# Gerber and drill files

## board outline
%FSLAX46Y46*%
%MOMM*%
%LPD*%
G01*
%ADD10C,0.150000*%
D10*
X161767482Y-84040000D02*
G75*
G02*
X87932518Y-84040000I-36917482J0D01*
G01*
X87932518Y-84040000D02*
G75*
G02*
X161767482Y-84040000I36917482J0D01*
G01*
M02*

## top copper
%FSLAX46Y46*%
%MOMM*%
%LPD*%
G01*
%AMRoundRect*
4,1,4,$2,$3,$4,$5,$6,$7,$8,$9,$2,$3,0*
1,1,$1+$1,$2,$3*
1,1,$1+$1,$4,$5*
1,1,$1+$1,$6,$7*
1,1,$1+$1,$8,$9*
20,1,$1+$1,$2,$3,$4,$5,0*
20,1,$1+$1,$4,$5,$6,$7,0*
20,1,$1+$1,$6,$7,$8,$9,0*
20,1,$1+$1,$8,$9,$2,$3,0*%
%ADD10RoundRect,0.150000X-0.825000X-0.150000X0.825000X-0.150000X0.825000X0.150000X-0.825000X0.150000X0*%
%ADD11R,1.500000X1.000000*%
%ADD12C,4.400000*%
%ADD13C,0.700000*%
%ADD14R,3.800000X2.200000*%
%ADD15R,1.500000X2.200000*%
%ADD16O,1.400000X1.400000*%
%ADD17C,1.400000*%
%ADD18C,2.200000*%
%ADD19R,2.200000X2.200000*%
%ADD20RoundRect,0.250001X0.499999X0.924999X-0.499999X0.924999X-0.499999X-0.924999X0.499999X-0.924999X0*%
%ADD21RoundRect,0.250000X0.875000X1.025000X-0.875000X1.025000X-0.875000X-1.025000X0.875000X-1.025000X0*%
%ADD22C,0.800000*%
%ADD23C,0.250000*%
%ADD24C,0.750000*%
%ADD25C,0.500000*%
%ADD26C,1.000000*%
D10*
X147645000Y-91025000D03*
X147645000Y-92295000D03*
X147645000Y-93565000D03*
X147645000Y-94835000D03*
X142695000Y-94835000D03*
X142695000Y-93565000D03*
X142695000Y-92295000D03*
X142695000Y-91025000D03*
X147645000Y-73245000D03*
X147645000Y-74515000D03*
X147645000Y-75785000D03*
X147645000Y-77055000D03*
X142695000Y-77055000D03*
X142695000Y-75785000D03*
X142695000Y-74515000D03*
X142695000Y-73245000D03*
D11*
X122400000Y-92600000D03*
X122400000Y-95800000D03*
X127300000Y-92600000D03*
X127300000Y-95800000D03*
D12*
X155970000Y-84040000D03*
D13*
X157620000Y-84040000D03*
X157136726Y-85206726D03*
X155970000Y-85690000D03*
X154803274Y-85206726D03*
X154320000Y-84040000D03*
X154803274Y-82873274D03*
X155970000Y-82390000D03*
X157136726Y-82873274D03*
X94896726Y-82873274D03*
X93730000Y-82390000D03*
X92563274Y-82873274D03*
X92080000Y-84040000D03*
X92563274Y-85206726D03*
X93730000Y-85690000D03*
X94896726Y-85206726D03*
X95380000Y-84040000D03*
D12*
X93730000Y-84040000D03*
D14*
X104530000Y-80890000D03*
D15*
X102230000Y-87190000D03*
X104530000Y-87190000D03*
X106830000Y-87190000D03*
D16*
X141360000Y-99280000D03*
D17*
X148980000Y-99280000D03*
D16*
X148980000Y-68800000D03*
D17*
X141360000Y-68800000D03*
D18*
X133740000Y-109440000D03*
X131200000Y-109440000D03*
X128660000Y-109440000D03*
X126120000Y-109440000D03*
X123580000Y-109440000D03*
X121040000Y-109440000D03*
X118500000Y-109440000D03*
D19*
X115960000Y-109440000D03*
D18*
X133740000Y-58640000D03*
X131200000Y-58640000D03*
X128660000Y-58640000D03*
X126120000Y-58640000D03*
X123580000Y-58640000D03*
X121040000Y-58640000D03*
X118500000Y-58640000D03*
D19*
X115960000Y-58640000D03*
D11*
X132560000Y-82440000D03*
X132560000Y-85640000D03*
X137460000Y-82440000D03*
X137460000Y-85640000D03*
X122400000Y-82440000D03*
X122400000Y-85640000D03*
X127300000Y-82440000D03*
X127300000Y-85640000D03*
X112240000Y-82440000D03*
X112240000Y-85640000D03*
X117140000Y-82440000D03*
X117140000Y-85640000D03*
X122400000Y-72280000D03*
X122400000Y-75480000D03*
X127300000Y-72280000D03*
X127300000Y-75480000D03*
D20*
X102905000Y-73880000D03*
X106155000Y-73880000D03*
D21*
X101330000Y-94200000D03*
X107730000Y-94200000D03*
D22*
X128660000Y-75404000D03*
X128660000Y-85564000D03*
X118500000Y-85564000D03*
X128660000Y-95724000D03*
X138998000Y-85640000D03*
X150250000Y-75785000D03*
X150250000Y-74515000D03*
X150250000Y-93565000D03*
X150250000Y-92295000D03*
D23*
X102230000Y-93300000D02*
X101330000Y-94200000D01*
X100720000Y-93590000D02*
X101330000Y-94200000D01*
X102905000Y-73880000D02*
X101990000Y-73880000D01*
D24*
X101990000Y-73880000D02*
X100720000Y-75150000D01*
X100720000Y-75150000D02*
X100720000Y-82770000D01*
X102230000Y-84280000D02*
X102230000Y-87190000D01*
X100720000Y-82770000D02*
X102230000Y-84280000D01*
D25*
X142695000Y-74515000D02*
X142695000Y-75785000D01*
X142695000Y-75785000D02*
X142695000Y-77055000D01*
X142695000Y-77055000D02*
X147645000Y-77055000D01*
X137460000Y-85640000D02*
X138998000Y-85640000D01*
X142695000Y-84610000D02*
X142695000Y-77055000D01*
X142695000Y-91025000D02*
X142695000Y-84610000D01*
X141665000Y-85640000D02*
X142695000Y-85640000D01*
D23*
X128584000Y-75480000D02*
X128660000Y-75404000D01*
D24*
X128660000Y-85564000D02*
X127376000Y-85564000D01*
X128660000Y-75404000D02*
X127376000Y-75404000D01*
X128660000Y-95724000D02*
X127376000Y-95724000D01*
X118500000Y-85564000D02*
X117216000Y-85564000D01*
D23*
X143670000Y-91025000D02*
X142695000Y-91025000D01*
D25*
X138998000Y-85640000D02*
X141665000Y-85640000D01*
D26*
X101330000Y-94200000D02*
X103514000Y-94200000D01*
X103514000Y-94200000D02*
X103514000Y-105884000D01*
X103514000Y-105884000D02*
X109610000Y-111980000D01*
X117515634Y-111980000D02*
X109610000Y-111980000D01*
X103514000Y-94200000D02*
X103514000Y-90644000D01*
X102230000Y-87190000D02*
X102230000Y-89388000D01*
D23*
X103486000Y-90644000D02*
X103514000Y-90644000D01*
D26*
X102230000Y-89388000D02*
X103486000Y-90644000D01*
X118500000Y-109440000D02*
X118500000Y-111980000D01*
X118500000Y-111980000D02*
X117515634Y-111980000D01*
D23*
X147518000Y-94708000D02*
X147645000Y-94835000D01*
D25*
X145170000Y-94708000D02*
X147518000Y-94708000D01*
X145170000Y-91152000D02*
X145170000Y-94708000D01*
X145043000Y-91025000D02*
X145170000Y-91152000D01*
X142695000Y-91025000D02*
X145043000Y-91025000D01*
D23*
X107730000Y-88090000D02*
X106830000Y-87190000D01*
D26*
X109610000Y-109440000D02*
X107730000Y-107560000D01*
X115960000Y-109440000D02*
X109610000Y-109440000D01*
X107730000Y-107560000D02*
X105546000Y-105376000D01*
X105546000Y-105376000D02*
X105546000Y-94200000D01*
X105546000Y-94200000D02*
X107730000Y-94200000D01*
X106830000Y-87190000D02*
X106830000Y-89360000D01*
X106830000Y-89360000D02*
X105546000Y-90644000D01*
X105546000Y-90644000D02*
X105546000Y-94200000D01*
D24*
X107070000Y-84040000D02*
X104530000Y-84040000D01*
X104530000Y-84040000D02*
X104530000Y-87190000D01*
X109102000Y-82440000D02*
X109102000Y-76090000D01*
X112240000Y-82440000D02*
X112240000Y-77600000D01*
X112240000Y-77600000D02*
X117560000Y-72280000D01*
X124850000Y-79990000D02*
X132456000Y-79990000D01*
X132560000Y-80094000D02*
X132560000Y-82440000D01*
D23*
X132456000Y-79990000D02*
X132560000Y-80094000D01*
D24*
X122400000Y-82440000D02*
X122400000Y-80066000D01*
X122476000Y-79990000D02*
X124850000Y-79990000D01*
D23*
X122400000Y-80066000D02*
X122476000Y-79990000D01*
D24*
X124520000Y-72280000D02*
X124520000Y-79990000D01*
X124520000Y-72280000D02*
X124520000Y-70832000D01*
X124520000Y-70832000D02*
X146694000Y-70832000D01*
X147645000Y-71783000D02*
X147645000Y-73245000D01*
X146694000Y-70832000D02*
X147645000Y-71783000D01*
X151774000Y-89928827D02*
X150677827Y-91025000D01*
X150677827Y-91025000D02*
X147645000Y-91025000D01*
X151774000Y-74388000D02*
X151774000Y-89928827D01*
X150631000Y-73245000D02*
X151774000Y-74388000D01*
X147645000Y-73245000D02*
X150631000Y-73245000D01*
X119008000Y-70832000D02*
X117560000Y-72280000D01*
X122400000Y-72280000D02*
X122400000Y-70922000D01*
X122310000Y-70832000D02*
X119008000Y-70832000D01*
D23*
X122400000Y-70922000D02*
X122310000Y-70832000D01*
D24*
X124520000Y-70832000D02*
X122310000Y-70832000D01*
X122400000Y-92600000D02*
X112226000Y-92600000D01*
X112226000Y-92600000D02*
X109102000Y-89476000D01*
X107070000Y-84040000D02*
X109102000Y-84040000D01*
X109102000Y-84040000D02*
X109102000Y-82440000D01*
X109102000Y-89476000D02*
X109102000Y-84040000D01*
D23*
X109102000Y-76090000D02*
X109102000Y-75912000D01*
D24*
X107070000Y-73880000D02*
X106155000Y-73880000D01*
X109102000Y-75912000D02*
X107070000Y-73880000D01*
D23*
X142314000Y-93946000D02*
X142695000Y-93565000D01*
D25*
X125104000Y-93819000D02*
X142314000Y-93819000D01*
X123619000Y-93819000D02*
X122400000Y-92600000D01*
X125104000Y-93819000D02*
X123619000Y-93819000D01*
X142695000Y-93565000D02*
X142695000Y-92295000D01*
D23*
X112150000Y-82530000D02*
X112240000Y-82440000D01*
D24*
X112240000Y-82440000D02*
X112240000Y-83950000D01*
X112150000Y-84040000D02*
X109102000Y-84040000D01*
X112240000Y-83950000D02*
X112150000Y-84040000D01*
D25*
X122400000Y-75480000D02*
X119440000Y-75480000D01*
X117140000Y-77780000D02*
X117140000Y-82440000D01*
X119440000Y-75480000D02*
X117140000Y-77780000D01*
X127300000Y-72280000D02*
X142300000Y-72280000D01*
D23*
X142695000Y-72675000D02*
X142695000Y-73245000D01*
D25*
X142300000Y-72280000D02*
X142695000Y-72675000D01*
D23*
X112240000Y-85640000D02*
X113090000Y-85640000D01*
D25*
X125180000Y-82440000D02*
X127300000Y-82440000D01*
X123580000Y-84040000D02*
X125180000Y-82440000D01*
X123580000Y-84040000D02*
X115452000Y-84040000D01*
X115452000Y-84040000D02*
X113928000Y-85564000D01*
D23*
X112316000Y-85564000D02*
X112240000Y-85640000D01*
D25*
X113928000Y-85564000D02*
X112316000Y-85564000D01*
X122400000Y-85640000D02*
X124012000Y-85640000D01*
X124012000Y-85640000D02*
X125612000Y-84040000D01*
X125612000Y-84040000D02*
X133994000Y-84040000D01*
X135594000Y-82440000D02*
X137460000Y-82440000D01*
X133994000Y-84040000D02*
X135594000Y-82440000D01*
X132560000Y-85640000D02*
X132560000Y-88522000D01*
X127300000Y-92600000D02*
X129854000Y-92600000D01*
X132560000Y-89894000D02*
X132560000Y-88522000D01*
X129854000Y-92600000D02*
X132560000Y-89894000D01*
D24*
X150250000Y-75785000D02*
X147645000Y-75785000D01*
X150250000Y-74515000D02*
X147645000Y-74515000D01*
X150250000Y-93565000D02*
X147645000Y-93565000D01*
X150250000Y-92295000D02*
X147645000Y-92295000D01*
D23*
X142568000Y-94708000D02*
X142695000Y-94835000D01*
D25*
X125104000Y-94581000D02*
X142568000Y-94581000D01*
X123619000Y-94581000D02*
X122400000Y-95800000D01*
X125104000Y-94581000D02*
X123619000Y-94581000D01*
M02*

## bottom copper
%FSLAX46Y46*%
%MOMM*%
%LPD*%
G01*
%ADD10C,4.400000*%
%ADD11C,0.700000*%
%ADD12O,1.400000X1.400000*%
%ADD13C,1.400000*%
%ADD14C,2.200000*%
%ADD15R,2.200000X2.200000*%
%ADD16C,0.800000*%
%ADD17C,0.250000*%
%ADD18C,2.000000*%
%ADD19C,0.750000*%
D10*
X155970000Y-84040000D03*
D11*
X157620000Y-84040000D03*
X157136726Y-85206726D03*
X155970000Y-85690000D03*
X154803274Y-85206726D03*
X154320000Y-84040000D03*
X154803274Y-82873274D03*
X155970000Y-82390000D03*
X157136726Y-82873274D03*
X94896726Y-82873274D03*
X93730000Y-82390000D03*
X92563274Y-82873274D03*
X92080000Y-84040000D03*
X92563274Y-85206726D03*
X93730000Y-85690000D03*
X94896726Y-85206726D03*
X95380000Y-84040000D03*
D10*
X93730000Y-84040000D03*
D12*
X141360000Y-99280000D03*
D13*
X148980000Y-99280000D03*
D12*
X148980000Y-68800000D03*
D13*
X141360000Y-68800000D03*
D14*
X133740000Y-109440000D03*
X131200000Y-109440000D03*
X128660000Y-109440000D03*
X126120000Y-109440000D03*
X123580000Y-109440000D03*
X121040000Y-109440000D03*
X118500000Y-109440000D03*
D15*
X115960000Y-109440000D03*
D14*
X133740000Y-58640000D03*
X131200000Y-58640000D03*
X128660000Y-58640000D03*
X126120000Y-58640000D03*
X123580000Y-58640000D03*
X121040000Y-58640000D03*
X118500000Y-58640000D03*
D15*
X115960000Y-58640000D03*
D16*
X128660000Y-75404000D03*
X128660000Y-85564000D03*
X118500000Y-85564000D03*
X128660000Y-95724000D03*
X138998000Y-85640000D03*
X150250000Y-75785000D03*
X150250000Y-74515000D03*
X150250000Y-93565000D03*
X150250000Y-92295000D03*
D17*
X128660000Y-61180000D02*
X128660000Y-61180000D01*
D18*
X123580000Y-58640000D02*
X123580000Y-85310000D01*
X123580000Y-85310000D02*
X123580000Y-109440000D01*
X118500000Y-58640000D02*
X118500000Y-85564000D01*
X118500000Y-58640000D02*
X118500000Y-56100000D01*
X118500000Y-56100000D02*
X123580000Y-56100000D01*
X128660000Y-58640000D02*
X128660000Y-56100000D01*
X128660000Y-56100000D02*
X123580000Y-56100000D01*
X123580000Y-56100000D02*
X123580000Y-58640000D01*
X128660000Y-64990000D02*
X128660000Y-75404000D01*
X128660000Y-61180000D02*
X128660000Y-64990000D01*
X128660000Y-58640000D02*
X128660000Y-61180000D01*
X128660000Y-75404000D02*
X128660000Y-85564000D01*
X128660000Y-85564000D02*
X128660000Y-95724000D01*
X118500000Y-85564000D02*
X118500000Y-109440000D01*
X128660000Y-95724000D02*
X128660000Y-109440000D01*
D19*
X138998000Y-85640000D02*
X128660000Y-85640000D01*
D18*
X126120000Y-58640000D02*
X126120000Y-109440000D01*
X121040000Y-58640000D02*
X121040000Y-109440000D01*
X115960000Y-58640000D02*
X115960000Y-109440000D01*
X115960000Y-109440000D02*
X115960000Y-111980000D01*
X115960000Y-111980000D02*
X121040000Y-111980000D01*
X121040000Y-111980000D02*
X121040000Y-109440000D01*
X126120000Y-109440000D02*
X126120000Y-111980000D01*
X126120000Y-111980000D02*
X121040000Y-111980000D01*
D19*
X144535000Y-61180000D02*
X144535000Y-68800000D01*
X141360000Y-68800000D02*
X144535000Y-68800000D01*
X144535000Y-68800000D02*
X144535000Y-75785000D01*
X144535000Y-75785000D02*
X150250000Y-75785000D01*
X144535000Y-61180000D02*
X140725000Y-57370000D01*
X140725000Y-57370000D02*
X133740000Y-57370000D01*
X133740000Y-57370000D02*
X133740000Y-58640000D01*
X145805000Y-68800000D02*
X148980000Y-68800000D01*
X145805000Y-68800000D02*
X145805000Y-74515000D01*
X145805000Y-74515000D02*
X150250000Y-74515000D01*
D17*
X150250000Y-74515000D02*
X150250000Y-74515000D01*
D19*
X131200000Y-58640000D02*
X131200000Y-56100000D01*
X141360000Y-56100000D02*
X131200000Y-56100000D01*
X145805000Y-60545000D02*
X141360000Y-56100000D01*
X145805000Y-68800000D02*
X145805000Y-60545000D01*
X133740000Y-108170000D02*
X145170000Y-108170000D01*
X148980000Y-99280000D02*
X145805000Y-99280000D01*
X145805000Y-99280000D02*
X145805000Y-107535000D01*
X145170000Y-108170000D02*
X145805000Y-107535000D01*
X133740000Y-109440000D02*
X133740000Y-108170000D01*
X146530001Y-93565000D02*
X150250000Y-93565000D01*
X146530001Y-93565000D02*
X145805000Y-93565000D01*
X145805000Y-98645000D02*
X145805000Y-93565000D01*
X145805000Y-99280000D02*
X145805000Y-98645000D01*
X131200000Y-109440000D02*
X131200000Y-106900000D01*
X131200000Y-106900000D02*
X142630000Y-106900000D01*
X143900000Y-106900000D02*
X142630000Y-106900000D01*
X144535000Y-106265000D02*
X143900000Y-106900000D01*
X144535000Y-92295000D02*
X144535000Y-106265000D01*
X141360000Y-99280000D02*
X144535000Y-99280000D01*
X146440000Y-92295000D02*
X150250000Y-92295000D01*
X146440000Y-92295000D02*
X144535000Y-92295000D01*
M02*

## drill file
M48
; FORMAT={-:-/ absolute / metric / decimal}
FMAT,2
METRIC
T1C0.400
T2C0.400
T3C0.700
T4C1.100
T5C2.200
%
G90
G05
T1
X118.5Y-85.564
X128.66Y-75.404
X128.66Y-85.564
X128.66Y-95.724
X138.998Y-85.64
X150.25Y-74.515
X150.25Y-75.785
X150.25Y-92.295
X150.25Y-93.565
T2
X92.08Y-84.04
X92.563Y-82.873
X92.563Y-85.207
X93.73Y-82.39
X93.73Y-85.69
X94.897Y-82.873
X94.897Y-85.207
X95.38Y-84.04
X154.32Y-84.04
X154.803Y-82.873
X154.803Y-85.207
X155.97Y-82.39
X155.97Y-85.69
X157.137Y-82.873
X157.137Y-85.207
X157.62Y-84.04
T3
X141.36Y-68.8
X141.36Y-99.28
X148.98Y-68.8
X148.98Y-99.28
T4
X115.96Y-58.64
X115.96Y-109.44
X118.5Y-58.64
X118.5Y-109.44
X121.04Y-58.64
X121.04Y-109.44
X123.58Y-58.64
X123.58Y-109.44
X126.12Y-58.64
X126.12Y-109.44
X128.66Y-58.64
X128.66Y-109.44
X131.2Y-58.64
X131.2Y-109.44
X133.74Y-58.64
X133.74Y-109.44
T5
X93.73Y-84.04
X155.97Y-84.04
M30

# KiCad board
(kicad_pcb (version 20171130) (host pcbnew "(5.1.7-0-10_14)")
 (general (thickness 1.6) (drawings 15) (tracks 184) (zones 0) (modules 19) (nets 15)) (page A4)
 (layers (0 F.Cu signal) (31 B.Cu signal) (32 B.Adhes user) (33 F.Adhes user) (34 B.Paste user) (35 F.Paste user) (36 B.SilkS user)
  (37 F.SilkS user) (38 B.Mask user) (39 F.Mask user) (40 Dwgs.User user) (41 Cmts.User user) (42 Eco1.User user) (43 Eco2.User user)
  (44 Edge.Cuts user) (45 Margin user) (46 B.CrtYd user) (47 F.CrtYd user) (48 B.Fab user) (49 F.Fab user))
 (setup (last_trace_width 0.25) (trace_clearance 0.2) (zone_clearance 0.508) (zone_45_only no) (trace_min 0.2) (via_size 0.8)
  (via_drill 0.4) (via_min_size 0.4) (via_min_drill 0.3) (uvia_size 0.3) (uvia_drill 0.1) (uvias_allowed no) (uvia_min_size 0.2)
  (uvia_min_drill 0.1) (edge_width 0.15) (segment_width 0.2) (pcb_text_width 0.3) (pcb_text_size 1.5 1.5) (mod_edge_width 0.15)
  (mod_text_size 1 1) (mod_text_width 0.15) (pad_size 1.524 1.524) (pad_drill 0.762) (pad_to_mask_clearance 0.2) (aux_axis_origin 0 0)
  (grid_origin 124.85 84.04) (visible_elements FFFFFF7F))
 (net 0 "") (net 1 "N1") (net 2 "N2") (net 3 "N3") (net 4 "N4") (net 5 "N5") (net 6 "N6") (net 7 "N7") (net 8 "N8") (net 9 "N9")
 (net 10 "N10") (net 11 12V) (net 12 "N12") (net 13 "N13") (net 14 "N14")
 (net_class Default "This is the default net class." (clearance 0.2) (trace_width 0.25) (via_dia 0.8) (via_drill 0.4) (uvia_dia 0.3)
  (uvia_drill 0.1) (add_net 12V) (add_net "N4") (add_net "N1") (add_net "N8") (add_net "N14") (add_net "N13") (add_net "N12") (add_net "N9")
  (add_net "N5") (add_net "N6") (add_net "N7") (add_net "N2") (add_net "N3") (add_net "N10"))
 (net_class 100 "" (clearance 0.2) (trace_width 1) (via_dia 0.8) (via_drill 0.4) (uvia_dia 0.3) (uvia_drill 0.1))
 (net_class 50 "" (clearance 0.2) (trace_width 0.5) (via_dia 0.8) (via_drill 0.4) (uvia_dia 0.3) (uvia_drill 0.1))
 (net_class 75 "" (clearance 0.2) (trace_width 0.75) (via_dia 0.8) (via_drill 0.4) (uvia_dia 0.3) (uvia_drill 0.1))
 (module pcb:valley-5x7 (layer F.Cu) (at 116.468 102.836)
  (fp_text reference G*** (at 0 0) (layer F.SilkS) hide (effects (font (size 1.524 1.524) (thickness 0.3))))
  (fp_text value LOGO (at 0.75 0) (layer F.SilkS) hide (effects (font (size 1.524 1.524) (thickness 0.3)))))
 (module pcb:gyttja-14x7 (layer F.Cu) (at 127.39 102.836)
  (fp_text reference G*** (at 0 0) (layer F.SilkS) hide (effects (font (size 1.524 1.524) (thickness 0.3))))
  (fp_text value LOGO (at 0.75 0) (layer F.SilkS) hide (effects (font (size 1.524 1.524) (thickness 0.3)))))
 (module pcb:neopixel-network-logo (layer F.Cu) (at 125.104 64.736)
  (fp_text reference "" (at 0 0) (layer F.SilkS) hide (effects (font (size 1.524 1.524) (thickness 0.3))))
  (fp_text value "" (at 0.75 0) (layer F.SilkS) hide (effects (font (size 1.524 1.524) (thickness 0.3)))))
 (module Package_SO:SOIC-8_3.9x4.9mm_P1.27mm (layer F.Cu) (at 145.17 92.93)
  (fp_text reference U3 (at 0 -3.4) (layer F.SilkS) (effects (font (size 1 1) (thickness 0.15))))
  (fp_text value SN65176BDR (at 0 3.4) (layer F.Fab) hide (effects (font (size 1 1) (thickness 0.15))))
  (pad 8 smd roundrect (at 2.475 -1.905) (size 1.95 0.6) (layers F.Cu F.Paste F.Mask) (roundrect_rratio 0.25) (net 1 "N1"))
  (pad 7 smd roundrect (at 2.475 -0.635) (size 1.95 0.6) (layers F.Cu F.Paste F.Mask) (roundrect_rratio 0.25) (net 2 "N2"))
  (pad 6 smd roundrect (at 2.475 0.635) (size 1.95 0.6) (layers F.Cu F.Paste F.Mask) (roundrect_rratio 0.25) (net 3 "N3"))
  (pad 5 smd roundrect (at 2.475 1.905) (size 1.95 0.6) (layers F.Cu F.Paste F.Mask) (roundrect_rratio 0.25) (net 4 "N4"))
  (pad 4 smd roundrect (at -2.475 1.905) (size 1.95 0.6) (layers F.Cu F.Paste F.Mask) (roundrect_rratio 0.25) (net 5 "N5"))
  (pad 3 smd roundrect (at -2.475 0.635) (size 1.95 0.6) (layers F.Cu F.Paste F.Mask) (roundrect_rratio 0.25) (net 1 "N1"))
  (pad 2 smd roundrect (at -2.475 -0.635) (size 1.95 0.6) (layers F.Cu F.Paste F.Mask) (roundrect_rratio 0.25) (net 1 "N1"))
  (pad 1 smd roundrect (at -2.475 -1.905) (size 1.95 0.6) (layers F.Cu F.Paste F.Mask) (roundrect_rratio 0.25) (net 4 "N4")))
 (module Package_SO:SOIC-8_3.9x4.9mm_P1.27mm (layer F.Cu) (at 145.17 75.15)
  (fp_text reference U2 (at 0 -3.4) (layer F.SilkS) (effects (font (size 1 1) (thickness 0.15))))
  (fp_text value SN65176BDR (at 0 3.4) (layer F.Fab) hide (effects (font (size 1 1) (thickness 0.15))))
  (pad 8 smd roundrect (at 2.475 -1.905) (size 1.95 0.6) (layers F.Cu F.Paste F.Mask) (roundrect_rratio 0.25) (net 1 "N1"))
  (pad 7 smd roundrect (at 2.475 -0.635) (size 1.95 0.6) (layers F.Cu F.Paste F.Mask) (roundrect_rratio 0.25) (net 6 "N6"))
  (pad 6 smd roundrect (at 2.475 0.635) (size 1.95 0.6) (layers F.Cu F.Paste F.Mask) (roundrect_rratio 0.25) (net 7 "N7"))
  (pad 5 smd roundrect (at 2.475 1.905) (size 1.95 0.6) (layers F.Cu F.Paste F.Mask) (roundrect_rratio 0.25) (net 4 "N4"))
  (pad 4 smd roundrect (at -2.475 1.905) (size 1.95 0.6) (layers F.Cu F.Paste F.Mask) (roundrect_rratio 0.25) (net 4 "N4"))
  (pad 3 smd roundrect (at -2.475 0.635) (size 1.95 0.6) (layers F.Cu F.Paste F.Mask) (roundrect_rratio 0.25) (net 4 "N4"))
  (pad 2 smd roundrect (at -2.475 -0.635) (size 1.95 0.6) (layers F.Cu F.Paste F.Mask) (roundrect_rratio 0.25) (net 4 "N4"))
  (pad 1 smd roundrect (at -2.475 -1.905) (size 1.95 0.6) (layers F.Cu F.Paste F.Mask) (roundrect_rratio 0.25) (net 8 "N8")))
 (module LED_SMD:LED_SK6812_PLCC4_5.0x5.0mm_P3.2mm (layer F.Cu) (at 124.85 94.2)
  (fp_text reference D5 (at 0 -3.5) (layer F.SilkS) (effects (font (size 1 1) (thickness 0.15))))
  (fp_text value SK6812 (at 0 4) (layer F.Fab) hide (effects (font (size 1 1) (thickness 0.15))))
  (pad 3 smd rect (at -2.45 -1.6) (size 1.5 1) (layers F.Cu F.Paste F.Mask) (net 1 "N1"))
  (pad 4 smd rect (at -2.45 1.6) (size 1.5 1) (layers F.Cu F.Paste F.Mask) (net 5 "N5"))
  (pad 2 smd rect (at 2.45 -1.6) (size 1.5 1) (layers F.Cu F.Paste F.Mask) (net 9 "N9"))
  (pad 1 smd rect (at 2.45 1.6) (size 1.5 1) (layers F.Cu F.Paste F.Mask) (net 4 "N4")))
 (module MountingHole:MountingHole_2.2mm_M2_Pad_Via (layer F.Cu) (at 155.97 84.04)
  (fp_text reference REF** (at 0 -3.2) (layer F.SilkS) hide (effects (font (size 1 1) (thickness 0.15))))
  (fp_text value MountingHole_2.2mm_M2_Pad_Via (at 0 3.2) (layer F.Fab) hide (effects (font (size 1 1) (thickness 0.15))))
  (pad 1 thru_hole circle (at 0 0) (size 4.4 4.4) (drill 2.2) (layers *.Cu *.Mask))
  (pad 1 thru_hole circle (at 1.65 0) (size 0.7 0.7) (drill 0.4) (layers *.Cu *.Mask))
  (pad 1 thru_hole circle (at 1.166726 1.166726) (size 0.7 0.7) (drill 0.4) (layers *.Cu *.Mask))
  (pad 1 thru_hole circle (at 0 1.65) (size 0.7 0.7) (drill 0.4) (layers *.Cu *.Mask))
  (pad 1 thru_hole circle (at -1.166726 1.166726) (size 0.7 0.7) (drill 0.4) (layers *.Cu *.Mask))
  (pad 1 thru_hole circle (at -1.65 0) (size 0.7 0.7) (drill 0.4) (layers *.Cu *.Mask))
  (pad 1 thru_hole circle (at -1.166726 -1.166726) (size 0.7 0.7) (drill 0.4) (layers *.Cu *.Mask))
  (pad 1 thru_hole circle (at 0 -1.65) (size 0.7 0.7) (drill 0.4) (layers *.Cu *.Mask))
  (pad 1 thru_hole circle (at 1.166726 -1.166726) (size 0.7 0.7) (drill 0.4) (layers *.Cu *.Mask)))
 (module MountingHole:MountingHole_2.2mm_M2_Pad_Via (layer F.Cu) (at 93.73 84.04)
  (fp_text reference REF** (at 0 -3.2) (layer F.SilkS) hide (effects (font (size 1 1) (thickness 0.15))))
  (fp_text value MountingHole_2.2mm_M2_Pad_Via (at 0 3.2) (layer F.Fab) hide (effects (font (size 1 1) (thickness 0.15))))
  (pad 1 thru_hole circle (at 1.166726 -1.166726) (size 0.7 0.7) (drill 0.4) (layers *.Cu *.Mask))
  (pad 1 thru_hole circle (at 0 -1.65) (size 0.7 0.7) (drill 0.4) (layers *.Cu *.Mask))
  (pad 1 thru_hole circle (at -1.166726 -1.166726) (size 0.7 0.7) (drill 0.4) (layers *.Cu *.Mask))
  (pad 1 thru_hole circle (at -1.65 0) (size 0.7 0.7) (drill 0.4) (layers *.Cu *.Mask))
  (pad 1 thru_hole circle (at -1.166726 1.166726) (size 0.7 0.7) (drill 0.4) (layers *.Cu *.Mask))
  (pad 1 thru_hole circle (at 0 1.65) (size 0.7 0.7) (drill 0.4) (layers *.Cu *.Mask))
  (pad 1 thru_hole circle (at 1.166726 1.166726) (size 0.7 0.7) (drill 0.4) (layers *.Cu *.Mask))
  (pad 1 thru_hole circle (at 1.65 0) (size 0.7 0.7) (drill 0.4) (layers *.Cu *.Mask))
  (pad 1 thru_hole circle (at 0 0) (size 4.4 4.4) (drill 2.2) (layers *.Cu *.Mask)))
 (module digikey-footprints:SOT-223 (layer F.Cu) (at 104.53 84.04)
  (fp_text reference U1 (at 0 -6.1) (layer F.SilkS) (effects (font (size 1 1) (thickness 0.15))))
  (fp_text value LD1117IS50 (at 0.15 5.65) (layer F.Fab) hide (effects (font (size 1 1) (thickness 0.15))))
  (pad 4 smd rect (at 0 -3.15) (size 3.8 2.2) (layers F.Cu F.Paste F.Mask) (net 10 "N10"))
  (pad 1 smd rect (at -2.3 3.15) (size 1.5 2.2) (layers F.Cu F.Paste F.Mask) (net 4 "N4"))
  (pad 2 smd rect (at 0 3.15) (size 1.5 2.2) (layers F.Cu F.Paste F.Mask) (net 1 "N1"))
  (pad 3 smd rect (at 2.3 3.15) (size 1.5 2.2) (layers F.Cu F.Paste F.Mask) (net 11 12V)))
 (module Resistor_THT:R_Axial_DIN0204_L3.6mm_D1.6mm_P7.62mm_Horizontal (layer F.Cu) (at 148.98 99.28 180)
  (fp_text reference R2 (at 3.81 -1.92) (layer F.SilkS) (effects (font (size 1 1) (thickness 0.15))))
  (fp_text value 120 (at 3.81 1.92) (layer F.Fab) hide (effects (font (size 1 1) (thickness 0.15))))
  (pad 2 thru_hole oval (at 7.62 0 180) (size 1.4 1.4) (drill 0.7) (layers *.Cu *.Mask) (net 2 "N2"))
  (pad 1 thru_hole circle (at 0 0 180) (size 1.4 1.4) (drill 0.7) (layers *.Cu *.Mask) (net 3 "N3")))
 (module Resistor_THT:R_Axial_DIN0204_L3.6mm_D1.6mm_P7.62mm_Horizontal (layer F.Cu) (at 141.36 68.8)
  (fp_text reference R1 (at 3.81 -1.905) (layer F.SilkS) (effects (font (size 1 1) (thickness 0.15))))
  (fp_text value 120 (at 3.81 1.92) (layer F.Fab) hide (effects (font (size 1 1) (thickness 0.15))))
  (pad 2 thru_hole oval (at 7.62 0) (size 1.4 1.4) (drill 0.7) (layers *.Cu *.Mask) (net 6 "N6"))
  (pad 1 thru_hole circle (at 0 0) (size 1.4 1.4) (drill 0.7) (layers *.Cu *.Mask) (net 7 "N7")))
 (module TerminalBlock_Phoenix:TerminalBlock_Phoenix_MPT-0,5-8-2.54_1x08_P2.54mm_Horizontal (layer B.Cu) (at 115.96 109.44)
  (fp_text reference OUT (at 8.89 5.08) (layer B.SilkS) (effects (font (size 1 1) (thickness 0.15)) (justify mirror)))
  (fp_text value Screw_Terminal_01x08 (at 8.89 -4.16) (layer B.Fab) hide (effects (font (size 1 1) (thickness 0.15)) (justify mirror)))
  (pad 8 thru_hole circle (at 17.78 0) (size 2.2 2.2) (drill 1.1) (layers *.Cu *.Mask) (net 3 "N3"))
  (pad 7 thru_hole circle (at 15.24 0) (size 2.2 2.2) (drill 1.1) (layers *.Cu *.Mask) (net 2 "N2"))
  (pad 6 thru_hole circle (at 12.7 0) (size 2.2 2.2) (drill 1.1) (layers *.Cu *.Mask) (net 4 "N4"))
  (pad 5 thru_hole circle (at 10.16 0) (size 2.2 2.2) (drill 1.1) (layers *.Cu *.Mask) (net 11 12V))
  (pad 4 thru_hole circle (at 7.62 0) (size 2.2 2.2) (drill 1.1) (layers *.Cu *.Mask) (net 4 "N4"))
  (pad 3 thru_hole circle (at 5.08 0) (size 2.2 2.2) (drill 1.1) (layers *.Cu *.Mask) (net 11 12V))
  (pad 2 thru_hole circle (at 2.54 0) (size 2.2 2.2) (drill 1.1) (layers *.Cu *.Mask) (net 4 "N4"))
  (pad 1 thru_hole rect (at 0 0) (size 2.2 2.2) (drill 1.1) (layers *.Cu *.Mask) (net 11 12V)))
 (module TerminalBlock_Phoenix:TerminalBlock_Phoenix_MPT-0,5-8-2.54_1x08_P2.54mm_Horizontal (layer B.Cu) (at 115.96 58.64)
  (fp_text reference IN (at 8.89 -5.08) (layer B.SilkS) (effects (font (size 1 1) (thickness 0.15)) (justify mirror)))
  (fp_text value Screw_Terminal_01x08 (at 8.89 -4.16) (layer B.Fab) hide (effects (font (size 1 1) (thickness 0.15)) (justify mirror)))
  (pad 8 thru_hole circle (at 17.78 0) (size 2.2 2.2) (drill 1.1) (layers *.Cu *.Mask) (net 7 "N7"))
  (pad 7 thru_hole circle (at 15.24 0) (size 2.2 2.2) (drill 1.1) (layers *.Cu *.Mask) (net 6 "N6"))
  (pad 6 thru_hole circle (at 12.7 0) (size 2.2 2.2) (drill 1.1) (layers *.Cu *.Mask) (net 4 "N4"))
  (pad 5 thru_hole circle (at 10.16 0) (size 2.2 2.2) (drill 1.1) (layers *.Cu *.Mask) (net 11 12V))
  (pad 4 thru_hole circle (at 7.62 0) (size 2.2 2.2) (drill 1.1) (layers *.Cu *.Mask) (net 4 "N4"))
  (pad 3 thru_hole circle (at 5.08 0) (size 2.2 2.2) (drill 1.1) (layers *.Cu *.Mask) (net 11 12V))
  (pad 2 thru_hole circle (at 2.54 0) (size 2.2 2.2) (drill 1.1) (layers *.Cu *.Mask) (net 4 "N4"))
  (pad 1 thru_hole rect (at 0 0) (size 2.2 2.2) (drill 1.1) (layers *.Cu *.Mask) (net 11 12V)))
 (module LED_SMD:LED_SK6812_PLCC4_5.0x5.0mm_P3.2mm (layer F.Cu) (at 135.01 84.04)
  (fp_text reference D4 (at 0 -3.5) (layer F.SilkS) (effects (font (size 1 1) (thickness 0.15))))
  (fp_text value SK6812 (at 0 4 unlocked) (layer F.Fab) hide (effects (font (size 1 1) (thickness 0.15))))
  (pad 3 smd rect (at -2.45 -1.6) (size 1.5 1) (layers F.Cu F.Paste F.Mask) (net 1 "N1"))
  (pad 4 smd rect (at -2.45 1.6) (size 1.5 1) (layers F.Cu F.Paste F.Mask) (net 9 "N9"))
  (pad 2 smd rect (at 2.45 -1.6) (size 1.5 1) (layers F.Cu F.Paste F.Mask) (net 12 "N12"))
  (pad 1 smd rect (at 2.45 1.6) (size 1.5 1) (layers F.Cu F.Paste F.Mask) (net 4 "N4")))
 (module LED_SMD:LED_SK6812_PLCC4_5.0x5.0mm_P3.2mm (layer F.Cu) (at 124.85 84.04)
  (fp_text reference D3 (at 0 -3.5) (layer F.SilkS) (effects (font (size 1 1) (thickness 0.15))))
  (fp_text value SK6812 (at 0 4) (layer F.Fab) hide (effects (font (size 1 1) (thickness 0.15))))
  (pad 3 smd rect (at -2.45 -1.6) (size 1.5 1) (layers F.Cu F.Paste F.Mask) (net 1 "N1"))
  (pad 4 smd rect (at -2.45 1.6) (size 1.5 1) (layers F.Cu F.Paste F.Mask) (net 12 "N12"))
  (pad 2 smd rect (at 2.45 -1.6) (size 1.5 1) (layers F.Cu F.Paste F.Mask) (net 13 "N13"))
  (pad 1 smd rect (at 2.45 1.6) (size 1.5 1) (layers F.Cu F.Paste F.Mask) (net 4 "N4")))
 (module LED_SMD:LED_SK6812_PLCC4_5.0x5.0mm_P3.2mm (layer F.Cu) (at 114.69 84.04)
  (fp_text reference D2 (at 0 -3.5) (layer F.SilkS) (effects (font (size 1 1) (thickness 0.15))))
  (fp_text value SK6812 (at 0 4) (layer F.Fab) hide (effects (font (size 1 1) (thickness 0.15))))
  (pad 3 smd rect (at -2.45 -1.6) (size 1.5 1) (layers F.Cu F.Paste F.Mask) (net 1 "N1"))
  (pad 4 smd rect (at -2.45 1.6) (size 1.5 1) (layers F.Cu F.Paste F.Mask) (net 13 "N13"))
  (pad 2 smd rect (at 2.45 -1.6) (size 1.5 1) (layers F.Cu F.Paste F.Mask) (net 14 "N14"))
  (pad 1 smd rect (at 2.45 1.6) (size 1.5 1) (layers F.Cu F.Paste F.Mask) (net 4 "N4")))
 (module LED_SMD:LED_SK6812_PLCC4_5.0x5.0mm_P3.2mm (layer F.Cu) (at 124.85 73.88)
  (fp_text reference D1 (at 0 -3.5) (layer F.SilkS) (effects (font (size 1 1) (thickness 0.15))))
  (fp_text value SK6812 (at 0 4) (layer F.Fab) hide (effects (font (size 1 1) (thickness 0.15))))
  (pad 3 smd rect (at -2.45 -1.6) (size 1.5 1) (layers F.Cu F.Paste F.Mask) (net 1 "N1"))
  (pad 4 smd rect (at -2.45 1.6) (size 1.5 1) (layers F.Cu F.Paste F.Mask) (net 14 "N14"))
  (pad 2 smd rect (at 2.45 -1.6) (size 1.5 1) (layers F.Cu F.Paste F.Mask) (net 8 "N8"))
  (pad 1 smd rect (at 2.45 1.6) (size 1.5 1) (layers F.Cu F.Paste F.Mask) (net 4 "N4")))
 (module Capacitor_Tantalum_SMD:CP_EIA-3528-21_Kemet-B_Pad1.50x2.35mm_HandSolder (layer F.Cu) (at 104.53 73.88 180)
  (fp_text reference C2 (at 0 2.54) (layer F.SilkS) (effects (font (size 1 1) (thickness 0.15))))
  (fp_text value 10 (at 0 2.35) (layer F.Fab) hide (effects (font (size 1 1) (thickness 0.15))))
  (pad 2 smd roundrect (at 1.625 0 180) (size 1.5 2.35) (layers F.Cu F.Paste F.Mask) (roundrect_rratio 0.166667) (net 4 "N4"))
  (pad 1 smd roundrect (at -1.625 0 180) (size 1.5 2.35) (layers F.Cu F.Paste F.Mask) (roundrect_rratio 0.166667) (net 1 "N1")))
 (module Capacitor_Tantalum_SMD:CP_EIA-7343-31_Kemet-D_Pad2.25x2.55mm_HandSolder (layer F.Cu) (at 104.53 94.2 180)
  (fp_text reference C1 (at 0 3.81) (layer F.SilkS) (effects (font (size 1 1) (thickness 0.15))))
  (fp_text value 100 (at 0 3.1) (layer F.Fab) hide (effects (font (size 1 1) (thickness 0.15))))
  (pad 2 smd roundrect (at 3.2 0 180) (size 2.25 2.55) (layers F.Cu F.Paste F.Mask) (roundrect_rratio 0.111111) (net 4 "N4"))
  (pad 1 smd roundrect (at -3.2 0 180) (size 2.25 2.55) (layers F.Cu F.Paste F.Mask) (roundrect_rratio 0.111111) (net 11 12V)))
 (gr_circle (center 124.85 84.04) (end 161.68 86.58) (layer Edge.Cuts) (width 0.15))
 (segment (start 128.66 61.18) (end 128.66 61.18) (width 0.25) (layer B.Cu) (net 4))
 (segment (start 102.23 93.3) (end 101.33 94.2) (width 0.25) (layer F.Cu) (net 4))
 (segment (start 100.72 93.59) (end 101.33 94.2) (width 0.25) (layer F.Cu) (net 4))
 (segment (start 102.905 73.88) (end 101.99 73.88) (width 0.25) (layer F.Cu) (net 4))
 (segment (start 101.99 73.88) (end 100.72 75.15) (width 0.75) (layer F.Cu) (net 4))
 (segment (start 100.72 75.15) (end 100.72 82.77) (width 0.75) (layer F.Cu) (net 4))
 (segment (start 102.23 84.28) (end 102.23 87.19) (width 0.75) (layer F.Cu) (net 4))
 (segment (start 100.72 82.77) (end 102.23 84.28) (width 0.75) (layer F.Cu) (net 4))
 (segment (start 123.58 58.64) (end 123.58 85.31) (width 2) (layer B.Cu) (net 4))
 (segment (start 123.58 85.31) (end 123.58 109.44) (width 2) (layer B.Cu) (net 4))
 (segment (start 118.5 58.64) (end 118.5 85.564) (width 2) (layer B.Cu) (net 4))
 (segment (start 118.5 58.64) (end 118.5 56.1) (width 2) (layer B.Cu) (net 4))
 (segment (start 118.5 56.1) (end 123.58 56.1) (width 2) (layer B.Cu) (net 4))
 (segment (start 128.66 58.64) (end 128.66 56.1) (width 2) (layer B.Cu) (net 4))
 (segment (start 128.66 56.1) (end 123.58 56.1) (width 2) (layer B.Cu) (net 4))
 (segment (start 123.58 56.1) (end 123.58 58.64) (width 2) (layer B.Cu) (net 4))
 (segment (start 128.66 64.99) (end 128.66 75.404) (width 2) (layer B.Cu) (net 4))
 (segment (start 128.66 61.18) (end 128.66 64.99) (width 2) (layer B.Cu) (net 4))
 (segment (start 128.66 58.64) (end 128.66 61.18) (width 2) (layer B.Cu) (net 4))
 (segment (start 142.695 74.515) (end 142.695 75.785) (width 0.5) (layer F.Cu) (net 4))
 (segment (start 142.695 75.785) (end 142.695 77.055) (width 0.5) (layer F.Cu) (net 4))
 (segment (start 142.695 77.055) (end 147.645 77.055) (width 0.5) (layer F.Cu) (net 4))
 (segment (start 137.46 85.64) (end 138.998 85.64) (width 0.5) (layer F.Cu) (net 4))
 (segment (start 142.695 84.61) (end 142.695 77.055) (width 0.5) (layer F.Cu) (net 4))
 (segment (start 142.695 91.025) (end 142.695 84.61) (width 0.5) (layer F.Cu) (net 4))
 (segment (start 141.665 85.64) (end 142.695 85.64) (width 0.5) (layer F.Cu) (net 4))
 (segment (start 128.66 75.404) (end 128.66 85.564) (width 2) (layer B.Cu) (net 4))
 (via (at 128.66 75.404) (size 0.8) (drill 0.4) (layers F.Cu B.Cu) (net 4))
 (segment (start 128.66 85.564) (end 128.66 95.724) (width 2) (layer B.Cu) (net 4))
 (via (at 128.66 85.564) (size 0.8) (drill 0.4) (layers F.Cu B.Cu) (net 4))
 (segment (start 118.5 85.564) (end 118.5 109.44) (width 2) (layer B.Cu) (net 4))
 (via (at 118.5 85.564) (size 0.8) (drill 0.4) (layers F.Cu B.Cu) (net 4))
 (segment (start 128.66 95.724) (end 128.66 109.44) (width 2) (layer B.Cu) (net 4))
 (via (at 128.66 95.724) (size 0.8) (drill 0.4) (layers F.Cu B.Cu) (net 4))
 (segment (start 128.584 75.48) (end 128.66 75.404) (width 0.25) (layer F.Cu) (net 4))
 (segment (start 128.66 85.564) (end 127.376 85.564) (width 0.75) (layer F.Cu) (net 4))
 (segment (start 128.66 75.404) (end 127.376 75.404) (width 0.75) (layer F.Cu) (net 4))
 (segment (start 128.66 95.724) (end 127.376 95.724) (width 0.75) (layer F.Cu) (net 4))
 (segment (start 118.5 85.564) (end 117.216 85.564) (width 0.75) (layer F.Cu) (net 4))
 (segment (start 143.67 91.025) (end 142.695 91.025) (width 0.25) (layer F.Cu) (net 4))
 (segment (start 138.998 85.64) (end 141.665 85.64) (width 0.5) (layer F.Cu) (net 4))
 (via (at 138.998 85.64) (size 0.8) (drill 0.4) (layers F.Cu B.Cu) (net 4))
 (segment (start 138.998 85.64) (end 128.66 85.64) (width 0.75) (layer B.Cu) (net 4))
 (segment (start 101.33 94.2) (end 103.514 94.2) (width 1) (layer F.Cu) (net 4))
 (segment (start 103.514 94.2) (end 103.514 105.884) (width 1) (layer F.Cu) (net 4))
 (segment (start 103.514 105.884) (end 109.61 111.98) (width 1) (layer F.Cu) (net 4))
 (segment (start 117.515634 111.98) (end 109.61 111.98) (width 1) (layer F.Cu) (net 4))
 (segment (start 103.514 94.2) (end 103.514 90.644) (width 1) (layer F.Cu) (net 4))
 (segment (start 102.23 87.19) (end 102.23 89.388) (width 1) (layer F.Cu) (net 4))
 (segment (start 103.486 90.644) (end 103.514 90.644) (width 0.25) (layer F.Cu) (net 4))
 (segment (start 102.23 89.388) (end 103.486 90.644) (width 1) (layer F.Cu) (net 4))
 (segment (start 118.5 109.44) (end 118.5 111.98) (width 1) (layer F.Cu) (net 4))
 (segment (start 118.5 111.98) (end 117.515634 111.98) (width 1) (layer F.Cu) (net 4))
 (segment (start 147.518 94.708) (end 147.645 94.835) (width 0.25) (layer F.Cu) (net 4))
 (segment (start 145.17 94.708) (end 147.518 94.708) (width 0.5) (layer F.Cu) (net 4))
 (segment (start 145.17 91.152) (end 145.17 94.708) (width 0.5) (layer F.Cu) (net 4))
 (segment (start 145.043 91.025) (end 145.17 91.152) (width 0.5) (layer F.Cu) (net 4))
 (segment (start 142.695 91.025) (end 145.043 91.025) (width 0.5) (layer F.Cu) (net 4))
 (segment (start 107.73 88.09) (end 106.83 87.19) (width 0.25) (layer F.Cu) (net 11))
 (segment (start 126.12 58.64) (end 126.12 109.44) (width 2) (layer B.Cu) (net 11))
 (segment (start 109.61 109.44) (end 107.73 107.56) (width 1) (layer F.Cu) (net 11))
 (segment (start 115.96 109.44) (end 109.61 109.44) (width 1) (layer F.Cu) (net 11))
 (segment (start 121.04 58.64) (end 121.04 109.44) (width 2) (layer B.Cu) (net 11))
 (segment (start 115.96 58.64) (end 115.96 109.44) (width 2) (layer B.Cu) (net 11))
 (segment (start 115.96 109.44) (end 115.96 111.98) (width 2) (layer B.Cu) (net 11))
 (segment (start 115.96 111.98) (end 121.04 111.98) (width 2) (layer B.Cu) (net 11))
 (segment (start 121.04 111.98) (end 121.04 109.44) (width 2) (layer B.Cu) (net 11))
 (segment (start 126.12 109.44) (end 126.12 111.98) (width 2) (layer B.Cu) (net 11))
 (segment (start 126.12 111.98) (end 121.04 111.98) (width 2) (layer B.Cu) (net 11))
 (segment (start 107.73 107.56) (end 105.546 105.376) (width 1) (layer F.Cu) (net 11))
 (segment (start 105.546 105.376) (end 105.546 94.2) (width 1) (layer F.Cu) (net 11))
 (segment (start 105.546 94.2) (end 107.73 94.2) (width 1) (layer F.Cu) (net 11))
 (segment (start 106.83 87.19) (end 106.83 89.36) (width 1) (layer F.Cu) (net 11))
 (segment (start 106.83 89.36) (end 105.546 90.644) (width 1) (layer F.Cu) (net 11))
 (segment (start 105.546 90.644) (end 105.546 94.2) (width 1) (layer F.Cu) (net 11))
 (segment (start 107.07 84.04) (end 104.53 84.04) (width 0.75) (layer F.Cu) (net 1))
 (segment (start 104.53 84.04) (end 104.53 87.19) (width 0.75) (layer F.Cu) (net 1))
 (segment (start 109.102 82.44) (end 109.102 76.09) (width 0.75) (layer F.Cu) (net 1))
 (segment (start 112.24 82.44) (end 112.24 77.6) (width 0.75) (layer F.Cu) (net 1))
 (segment (start 112.24 77.6) (end 117.56 72.28) (width 0.75) (layer F.Cu) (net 1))
 (segment (start 124.85 79.99) (end 132.456 79.99) (width 0.75) (layer F.Cu) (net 1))
 (segment (start 132.56 80.094) (end 132.56 82.44) (width 0.75) (layer F.Cu) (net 1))
 (segment (start 132.456 79.99) (end 132.56 80.094) (width 0.25) (layer F.Cu) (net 1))
 (segment (start 122.4 82.44) (end 122.4 80.066) (width 0.75) (layer F.Cu) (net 1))
 (segment (start 122.476 79.99) (end 124.85 79.99) (width 0.75) (layer F.Cu) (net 1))
 (segment (start 122.4 80.066) (end 122.476 79.99) (width 0.25) (layer F.Cu) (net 1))
 (segment (start 124.52 72.28) (end 124.52 79.99) (width 0.75) (layer F.Cu) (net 1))
 (segment (start 124.52 72.28) (end 124.52 70.832) (width 0.75) (layer F.Cu) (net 1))
 (segment (start 124.52 70.832) (end 146.694 70.832) (width 0.75) (layer F.Cu) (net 1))
 (segment (start 147.645 71.783) (end 147.645 73.245) (width 0.75) (layer F.Cu) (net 1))
 (segment (start 146.694 70.832) (end 147.645 71.783) (width 0.75) (layer F.Cu) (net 1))
 (segment (start 151.774 89.928827) (end 150.677827 91.025) (width 0.75) (layer F.Cu) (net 1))
 (segment (start 150.677827 91.025) (end 147.645 91.025) (width 0.75) (layer F.Cu) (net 1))
 (segment (start 151.774 74.388) (end 151.774 89.928827) (width 0.75) (layer F.Cu) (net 1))
 (segment (start 150.631 73.245) (end 151.774 74.388) (width 0.75) (layer F.Cu) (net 1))
 (segment (start 147.645 73.245) (end 150.631 73.245) (width 0.75) (layer F.Cu) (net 1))
 (segment (start 119.008 70.832) (end 117.56 72.28) (width 0.75) (layer F.Cu) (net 1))
 (segment (start 122.4 72.28) (end 122.4 70.922) (width 0.75) (layer F.Cu) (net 1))
 (segment (start 122.31 70.832) (end 119.008 70.832) (width 0.75) (layer F.Cu) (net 1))
 (segment (start 122.4 70.922) (end 122.31 70.832) (width 0.25) (layer F.Cu) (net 1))
 (segment (start 124.52 70.832) (end 122.31 70.832) (width 0.75) (layer F.Cu) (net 1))
 (segment (start 122.4 92.6) (end 112.226 92.6) (width 0.75) (layer F.Cu) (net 1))
 (segment (start 112.226 92.6) (end 109.102 89.476) (width 0.75) (layer F.Cu) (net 1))
 (segment (start 107.07 84.04) (end 109.102 84.04) (width 0.75) (layer F.Cu) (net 1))
 (segment (start 109.102 84.04) (end 109.102 82.44) (width 0.75) (layer F.Cu) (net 1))
 (segment (start 109.102 89.476) (end 109.102 84.04) (width 0.75) (layer F.Cu) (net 1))
 (segment (start 109.102 76.09) (end 109.102 75.912) (width 0.25) (layer F.Cu) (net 1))
 (segment (start 107.07 73.88) (end 106.155 73.88) (width 0.75) (layer F.Cu) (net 1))
 (segment (start 109.102 75.912) (end 107.07 73.88) (width 0.75) (layer F.Cu) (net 1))
 (segment (start 142.314 93.946) (end 142.695 93.565) (width 0.25) (layer F.Cu) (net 1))
 (segment (start 125.104 93.819) (end 142.314 93.819) (width 0.5) (layer F.Cu) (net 1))
 (segment (start 123.619 93.819) (end 122.4 92.6) (width 0.5) (layer F.Cu) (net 1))
 (segment (start 125.104 93.819) (end 123.619 93.819) (width 0.5) (layer F.Cu) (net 1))
 (segment (start 142.695 93.565) (end 142.695 92.295) (width 0.5) (layer F.Cu) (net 1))
 (segment (start 112.15 82.53) (end 112.24 82.44) (width 0.25) (layer F.Cu) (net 1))
 (segment (start 112.24 82.44) (end 112.24 83.95) (width 0.75) (layer F.Cu) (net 1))
 (segment (start 112.15 84.04) (end 109.102 84.04) (width 0.75) (layer F.Cu) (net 1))
 (segment (start 112.24 83.95) (end 112.15 84.04) (width 0.75) (layer F.Cu) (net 1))
 (segment (start 122.4 75.48) (end 119.44 75.48) (width 0.5) (layer F.Cu) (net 14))
 (segment (start 117.14 77.78) (end 117.14 82.44) (width 0.5) (layer F.Cu) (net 14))
 (segment (start 119.44 75.48) (end 117.14 77.78) (width 0.5) (layer F.Cu) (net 14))
 (segment (start 127.3 72.28) (end 142.3 72.28) (width 0.5) (layer F.Cu) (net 8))
 (segment (start 142.695 72.675) (end 142.695 73.245) (width 0.25) (layer F.Cu) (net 8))
 (segment (start 142.3 72.28) (end 142.695 72.675) (width 0.5) (layer F.Cu) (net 8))
 (segment (start 112.24 85.64) (end 113.09 85.64) (width 0.25) (layer F.Cu) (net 13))
 (segment (start 125.18 82.44) (end 127.3 82.44) (width 0.5) (layer F.Cu) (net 13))
 (segment (start 123.58 84.04) (end 125.18 82.44) (width 0.5) (layer F.Cu) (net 13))
 (segment (start 123.58 84.04) (end 115.452 84.04) (width 0.5) (layer F.Cu) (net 13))
 (segment (start 115.452 84.04) (end 113.928 85.564) (width 0.5) (layer F.Cu) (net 13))
 (segment (start 112.316 85.564) (end 112.24 85.64) (width 0.25) (layer F.Cu) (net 13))
 (segment (start 113.928 85.564) (end 112.316 85.564) (width 0.5) (layer F.Cu) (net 13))
 (segment (start 122.4 85.64) (end 124.012 85.64) (width 0.5) (layer F.Cu) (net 12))
 (segment (start 124.012 85.64) (end 125.612 84.04) (width 0.5) (layer F.Cu) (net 12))
 (segment (start 125.612 84.04) (end 133.994 84.04) (width 0.5) (layer F.Cu) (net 12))
 (segment (start 135.594 82.44) (end 137.46 82.44) (width 0.5) (layer F.Cu) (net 12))
 (segment (start 133.994 84.04) (end 135.594 82.44) (width 0.5) (layer F.Cu) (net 12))
 (segment (start 132.56 85.64) (end 132.56 88.522) (width 0.5) (layer F.Cu) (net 9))
 (segment (start 127.3 92.6) (end 129.854 92.6) (width 0.5) (layer F.Cu) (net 9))
 (segment (start 132.56 89.894) (end 132.56 88.522) (width 0.5) (layer F.Cu) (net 9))
 (segment (start 129.854 92.6) (end 132.56 89.894) (width 0.5) (layer F.Cu) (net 9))
 (via (at 150.25 75.785) (size 0.8) (drill 0.4) (layers F.Cu B.Cu) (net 7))
 (segment (start 144.535 61.18) (end 144.535 68.8) (width 0.75) (layer B.Cu) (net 7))
 (segment (start 141.36 68.8) (end 144.535 68.8) (width 0.75) (layer B.Cu) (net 7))
 (segment (start 144.535 68.8) (end 144.535 75.785) (width 0.75) (layer B.Cu) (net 7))
 (segment (start 144.535 75.785) (end 150.25 75.785) (width 0.75) (layer B.Cu) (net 7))
 (segment (start 144.535 61.18) (end 140.725 57.37) (width 0.75) (layer B.Cu) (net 7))
 (segment (start 140.725 57.37) (end 133.74 57.37) (width 0.75) (layer B.Cu) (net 7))
 (segment (start 133.74 57.37) (end 133.74 58.64) (width 0.75) (layer B.Cu) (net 7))
 (segment (start 150.25 75.785) (end 147.645 75.785) (width 0.75) (layer F.Cu) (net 7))
 (segment (start 145.805 68.8) (end 148.98 68.8) (width 0.75) (layer B.Cu) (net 6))
 (segment (start 145.805 68.8) (end 145.805 74.515) (width 0.75) (layer B.Cu) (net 6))
 (segment (start 145.805 74.515) (end 150.25 74.515) (width 0.75) (layer B.Cu) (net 6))
 (segment (start 150.25 74.515) (end 150.25 74.515) (width 0.25) (layer B.Cu) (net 6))
 (via (at 150.25 74.515) (size 0.8) (drill 0.4) (layers F.Cu B.Cu) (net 6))
 (segment (start 150.25 74.515) (end 147.645 74.515) (width 0.75) (layer F.Cu) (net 6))
 (segment (start 131.2 58.64) (end 131.2 56.1) (width 0.75) (layer B.Cu) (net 6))
 (segment (start 141.36 56.1) (end 131.2 56.1) (width 0.75) (layer B.Cu) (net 6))
 (segment (start 145.805 60.545) (end 141.36 56.1) (width 0.75) (layer B.Cu) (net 6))
 (segment (start 145.805 68.8) (end 145.805 60.545) (width 0.75) (layer B.Cu) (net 6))
 (via (at 150.25 93.565) (size 0.8) (drill 0.4) (layers F.Cu B.Cu) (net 3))
 (segment (start 133.74 108.17) (end 145.17 108.17) (width 0.75) (layer B.Cu) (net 3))
 (segment (start 148.98 99.28) (end 145.805 99.28) (width 0.75) (layer B.Cu) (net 3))
 (segment (start 145.805 99.28) (end 145.805 107.535) (width 0.75) (layer B.Cu) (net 3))
 (segment (start 145.17 108.17) (end 145.805 107.535) (width 0.75) (layer B.Cu) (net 3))
 (segment (start 133.74 109.44) (end 133.74 108.17) (width 0.75) (layer B.Cu) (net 3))
 (segment (start 146.530001 93.565) (end 150.25 93.565) (width 0.75) (layer B.Cu) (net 3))
 (segment (start 146.530001 93.565) (end 145.805 93.565) (width 0.75) (layer B.Cu) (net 3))
 (segment (start 145.805 98.645) (end 145.805 93.565) (width 0.75) (layer B.Cu) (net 3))
 (segment (start 145.805 99.28) (end 145.805 98.645) (width 0.75) (layer B.Cu) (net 3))
 (segment (start 150.25 93.565) (end 147.645 93.565) (width 0.75) (layer F.Cu) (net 3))
 (via (at 150.25 92.295) (size 0.8) (drill 0.4) (layers F.Cu B.Cu) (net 2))
 (segment (start 131.2 109.44) (end 131.2 106.9) (width 0.75) (layer B.Cu) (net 2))
 (segment (start 131.2 106.9) (end 142.63 106.9) (width 0.75) (layer B.Cu) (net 2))
 (segment (start 143.9 106.9) (end 142.63 106.9) (width 0.75) (layer B.Cu) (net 2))
 (segment (start 144.535 106.265) (end 143.9 106.9) (width 0.75) (layer B.Cu) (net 2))
 (segment (start 144.535 92.295) (end 144.535 106.265) (width 0.75) (layer B.Cu) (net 2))
 (segment (start 141.36 99.28) (end 144.535 99.28) (width 0.75) (layer B.Cu) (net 2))
 (segment (start 146.44 92.295) (end 150.25 92.295) (width 0.75) (layer B.Cu) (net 2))
 (segment (start 146.44 92.295) (end 144.535 92.295) (width 0.75) (layer B.Cu) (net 2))
 (segment (start 150.25 92.295) (end 147.645 92.295) (width 0.75) (layer F.Cu) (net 2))
 (segment (start 142.568 94.708) (end 142.695 94.835) (width 0.25) (layer F.Cu) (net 5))
 (segment (start 125.104 94.581) (end 142.568 94.581) (width 0.5) (layer F.Cu) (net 5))
 (segment (start 123.619 94.581) (end 122.4 95.8) (width 0.5) (layer F.Cu) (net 5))
 (segment (start 125.104 94.581) (end 123.619 94.581) (width 0.5) (layer F.Cu) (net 5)))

